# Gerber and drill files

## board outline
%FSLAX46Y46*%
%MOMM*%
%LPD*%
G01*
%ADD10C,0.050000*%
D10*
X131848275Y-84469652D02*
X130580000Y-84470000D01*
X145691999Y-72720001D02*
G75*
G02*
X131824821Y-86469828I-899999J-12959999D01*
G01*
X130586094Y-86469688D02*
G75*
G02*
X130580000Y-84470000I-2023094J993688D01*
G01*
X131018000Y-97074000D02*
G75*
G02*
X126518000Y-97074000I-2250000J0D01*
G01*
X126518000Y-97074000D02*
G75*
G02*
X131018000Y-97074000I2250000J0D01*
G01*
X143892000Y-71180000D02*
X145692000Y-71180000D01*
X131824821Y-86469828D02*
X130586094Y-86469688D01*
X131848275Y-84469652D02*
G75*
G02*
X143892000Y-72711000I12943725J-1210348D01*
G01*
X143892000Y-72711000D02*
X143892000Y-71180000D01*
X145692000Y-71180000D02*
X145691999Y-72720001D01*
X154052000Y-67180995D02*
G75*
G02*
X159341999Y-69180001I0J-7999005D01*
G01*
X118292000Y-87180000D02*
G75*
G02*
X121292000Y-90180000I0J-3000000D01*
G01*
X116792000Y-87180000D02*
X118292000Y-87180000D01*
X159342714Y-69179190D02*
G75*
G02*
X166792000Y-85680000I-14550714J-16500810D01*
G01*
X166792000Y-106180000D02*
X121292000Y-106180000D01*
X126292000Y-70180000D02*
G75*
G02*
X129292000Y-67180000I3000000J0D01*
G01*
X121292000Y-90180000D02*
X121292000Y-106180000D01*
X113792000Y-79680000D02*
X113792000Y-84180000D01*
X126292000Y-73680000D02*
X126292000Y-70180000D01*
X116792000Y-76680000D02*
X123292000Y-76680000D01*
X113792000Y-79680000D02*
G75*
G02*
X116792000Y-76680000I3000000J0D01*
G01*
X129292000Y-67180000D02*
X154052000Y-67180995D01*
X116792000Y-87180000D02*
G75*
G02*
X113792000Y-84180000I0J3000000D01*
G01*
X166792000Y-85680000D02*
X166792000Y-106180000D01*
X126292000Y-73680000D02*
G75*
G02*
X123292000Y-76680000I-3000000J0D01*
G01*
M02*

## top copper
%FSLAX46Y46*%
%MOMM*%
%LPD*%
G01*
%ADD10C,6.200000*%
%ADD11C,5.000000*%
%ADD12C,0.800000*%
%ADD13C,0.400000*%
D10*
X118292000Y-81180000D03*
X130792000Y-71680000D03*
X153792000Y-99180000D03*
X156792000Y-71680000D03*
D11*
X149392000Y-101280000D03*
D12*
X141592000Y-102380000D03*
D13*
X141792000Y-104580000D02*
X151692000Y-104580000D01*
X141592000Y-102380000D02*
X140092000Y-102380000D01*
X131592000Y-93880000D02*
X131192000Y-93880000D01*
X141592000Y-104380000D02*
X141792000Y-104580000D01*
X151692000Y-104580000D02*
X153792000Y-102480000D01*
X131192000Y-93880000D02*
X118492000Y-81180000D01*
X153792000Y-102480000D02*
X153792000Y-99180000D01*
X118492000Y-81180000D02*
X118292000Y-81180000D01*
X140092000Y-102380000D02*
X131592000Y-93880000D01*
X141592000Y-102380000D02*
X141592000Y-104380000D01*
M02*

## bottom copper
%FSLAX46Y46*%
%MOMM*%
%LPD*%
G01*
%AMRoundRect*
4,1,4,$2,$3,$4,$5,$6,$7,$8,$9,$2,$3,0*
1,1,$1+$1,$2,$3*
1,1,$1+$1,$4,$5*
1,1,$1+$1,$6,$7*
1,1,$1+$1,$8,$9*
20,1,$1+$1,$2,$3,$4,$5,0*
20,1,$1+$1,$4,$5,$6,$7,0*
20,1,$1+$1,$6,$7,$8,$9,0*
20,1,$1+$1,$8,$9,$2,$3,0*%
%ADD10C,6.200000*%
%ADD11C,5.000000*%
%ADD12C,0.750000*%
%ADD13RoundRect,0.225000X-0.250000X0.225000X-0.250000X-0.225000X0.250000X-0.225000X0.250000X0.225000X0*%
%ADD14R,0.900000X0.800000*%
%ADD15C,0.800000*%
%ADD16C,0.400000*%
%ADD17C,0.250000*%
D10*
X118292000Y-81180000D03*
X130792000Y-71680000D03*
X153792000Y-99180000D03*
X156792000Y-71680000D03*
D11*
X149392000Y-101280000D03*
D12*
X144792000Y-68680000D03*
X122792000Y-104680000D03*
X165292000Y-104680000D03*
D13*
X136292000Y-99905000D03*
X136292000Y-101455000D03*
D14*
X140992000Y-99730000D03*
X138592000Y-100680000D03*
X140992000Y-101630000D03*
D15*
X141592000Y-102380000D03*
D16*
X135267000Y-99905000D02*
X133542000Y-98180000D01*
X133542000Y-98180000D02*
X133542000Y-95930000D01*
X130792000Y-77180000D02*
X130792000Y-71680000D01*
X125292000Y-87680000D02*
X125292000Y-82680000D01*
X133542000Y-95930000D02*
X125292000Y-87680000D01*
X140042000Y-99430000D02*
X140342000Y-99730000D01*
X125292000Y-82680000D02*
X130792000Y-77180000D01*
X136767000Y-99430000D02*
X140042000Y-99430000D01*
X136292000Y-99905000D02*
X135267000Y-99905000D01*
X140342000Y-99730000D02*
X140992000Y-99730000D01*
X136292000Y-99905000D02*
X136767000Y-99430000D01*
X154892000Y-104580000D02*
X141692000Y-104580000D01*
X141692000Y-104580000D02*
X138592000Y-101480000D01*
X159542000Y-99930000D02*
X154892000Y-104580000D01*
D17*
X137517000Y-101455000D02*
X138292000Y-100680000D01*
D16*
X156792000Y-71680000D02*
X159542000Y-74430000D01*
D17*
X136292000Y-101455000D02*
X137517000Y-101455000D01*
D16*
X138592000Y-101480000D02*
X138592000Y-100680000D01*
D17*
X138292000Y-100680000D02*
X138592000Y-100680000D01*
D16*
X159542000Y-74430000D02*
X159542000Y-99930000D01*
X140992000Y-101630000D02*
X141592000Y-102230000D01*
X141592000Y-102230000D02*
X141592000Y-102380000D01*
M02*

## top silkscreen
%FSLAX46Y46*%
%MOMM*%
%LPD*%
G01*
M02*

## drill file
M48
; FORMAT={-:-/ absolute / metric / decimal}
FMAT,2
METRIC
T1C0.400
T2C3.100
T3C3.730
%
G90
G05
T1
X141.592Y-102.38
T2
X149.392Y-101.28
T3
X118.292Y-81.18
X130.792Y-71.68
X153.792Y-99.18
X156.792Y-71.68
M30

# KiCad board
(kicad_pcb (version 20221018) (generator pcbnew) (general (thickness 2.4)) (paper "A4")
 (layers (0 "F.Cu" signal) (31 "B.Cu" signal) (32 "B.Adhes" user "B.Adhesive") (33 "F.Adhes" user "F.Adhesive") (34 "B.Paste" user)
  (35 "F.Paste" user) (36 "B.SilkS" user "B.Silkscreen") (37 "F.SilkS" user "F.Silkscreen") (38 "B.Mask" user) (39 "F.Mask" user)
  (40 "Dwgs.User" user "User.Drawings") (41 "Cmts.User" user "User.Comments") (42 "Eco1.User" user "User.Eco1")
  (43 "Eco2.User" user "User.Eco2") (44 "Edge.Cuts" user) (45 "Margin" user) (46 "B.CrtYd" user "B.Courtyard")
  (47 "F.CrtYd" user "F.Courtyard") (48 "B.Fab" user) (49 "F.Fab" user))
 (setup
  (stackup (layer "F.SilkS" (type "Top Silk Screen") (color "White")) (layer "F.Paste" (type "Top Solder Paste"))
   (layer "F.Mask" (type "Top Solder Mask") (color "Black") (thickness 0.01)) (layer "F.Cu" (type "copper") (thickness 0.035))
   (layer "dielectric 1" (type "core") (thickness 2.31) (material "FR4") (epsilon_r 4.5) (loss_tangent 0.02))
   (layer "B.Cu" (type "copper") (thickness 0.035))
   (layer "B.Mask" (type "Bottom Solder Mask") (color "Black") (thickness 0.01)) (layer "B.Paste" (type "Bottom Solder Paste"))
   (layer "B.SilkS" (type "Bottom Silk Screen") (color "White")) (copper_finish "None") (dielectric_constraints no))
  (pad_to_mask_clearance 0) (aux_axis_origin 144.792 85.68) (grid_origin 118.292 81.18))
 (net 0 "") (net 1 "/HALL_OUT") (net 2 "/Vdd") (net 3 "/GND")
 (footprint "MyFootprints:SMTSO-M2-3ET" (layer "F.Cu") (at 118.292 81.18 180)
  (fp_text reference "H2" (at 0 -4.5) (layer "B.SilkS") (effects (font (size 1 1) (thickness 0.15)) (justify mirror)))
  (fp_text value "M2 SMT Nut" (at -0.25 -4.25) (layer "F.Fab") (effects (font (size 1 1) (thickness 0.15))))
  (pad "1" thru_hole circle (at 0 0 180) (size 6.2 6.2) (drill 3.73) (layers "*.Cu" "*.Mask" "B.Paste") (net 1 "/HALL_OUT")))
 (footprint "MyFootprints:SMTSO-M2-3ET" (layer "F.Cu") (at 130.792 71.68 180)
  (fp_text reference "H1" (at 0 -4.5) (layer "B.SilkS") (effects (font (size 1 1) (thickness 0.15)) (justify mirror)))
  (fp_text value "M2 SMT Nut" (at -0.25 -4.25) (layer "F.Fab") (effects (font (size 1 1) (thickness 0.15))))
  (pad "1" thru_hole circle (at 0 0 180) (size 6.2 6.2) (drill 3.73) (layers "*.Cu" "*.Mask" "B.Paste") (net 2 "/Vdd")))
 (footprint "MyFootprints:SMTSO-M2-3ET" (layer "F.Cu") (at 153.792 99.18 180)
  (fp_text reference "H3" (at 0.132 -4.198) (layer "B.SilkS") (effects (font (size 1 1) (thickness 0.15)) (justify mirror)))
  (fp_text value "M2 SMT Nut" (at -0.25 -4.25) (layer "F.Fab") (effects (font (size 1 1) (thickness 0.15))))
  (pad "1" thru_hole circle (at 0 0 180) (size 6.2 6.2) (drill 3.73) (layers "*.Cu" "*.Mask" "B.Paste") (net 1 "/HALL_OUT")))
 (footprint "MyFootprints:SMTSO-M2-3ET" (layer "F.Cu") (at 156.792 71.68 180)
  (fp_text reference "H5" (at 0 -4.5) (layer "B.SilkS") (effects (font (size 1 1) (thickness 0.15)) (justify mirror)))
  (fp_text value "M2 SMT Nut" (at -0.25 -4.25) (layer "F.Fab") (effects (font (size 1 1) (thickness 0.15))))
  (pad "1" thru_hole circle (at 0 0 180) (size 6.2 6.2) (drill 3.73) (layers "*.Cu" "*.Mask" "B.Paste") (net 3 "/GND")))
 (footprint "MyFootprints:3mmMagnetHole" (layer "F.Cu") (at 149.392 101.28)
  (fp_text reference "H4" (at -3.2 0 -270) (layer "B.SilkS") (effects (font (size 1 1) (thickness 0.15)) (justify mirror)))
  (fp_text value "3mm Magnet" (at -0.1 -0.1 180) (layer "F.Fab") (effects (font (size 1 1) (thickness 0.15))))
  (pad "1" thru_hole circle (at 0 0) (size 5 5) (drill 3.1) (layers "*.Cu" "*.Mask" "F.Paste")))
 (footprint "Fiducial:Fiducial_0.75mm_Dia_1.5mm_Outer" (layer "B.Cu") (at 144.792 68.68)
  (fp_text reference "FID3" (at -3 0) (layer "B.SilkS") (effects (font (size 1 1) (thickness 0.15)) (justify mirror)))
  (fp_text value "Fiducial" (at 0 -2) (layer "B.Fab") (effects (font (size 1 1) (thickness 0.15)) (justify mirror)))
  (pad "" smd circle (at 0 0) (size 0.75 0.75) (layers "B.Cu" "B.Mask") (solder_mask_margin 0.375) (clearance 0.375)))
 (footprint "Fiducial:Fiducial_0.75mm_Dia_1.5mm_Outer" (layer "B.Cu") (at 122.792 104.68)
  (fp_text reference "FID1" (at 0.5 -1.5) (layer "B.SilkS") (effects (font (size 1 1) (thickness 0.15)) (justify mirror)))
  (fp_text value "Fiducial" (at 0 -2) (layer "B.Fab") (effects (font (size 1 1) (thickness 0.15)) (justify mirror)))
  (pad "" smd circle (at 0 0) (size 0.75 0.75) (layers "B.Cu" "B.Mask") (solder_mask_margin 0.375) (clearance 0.375)))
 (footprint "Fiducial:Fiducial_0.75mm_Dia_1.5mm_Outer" (layer "B.Cu") (at 165.292 104.68)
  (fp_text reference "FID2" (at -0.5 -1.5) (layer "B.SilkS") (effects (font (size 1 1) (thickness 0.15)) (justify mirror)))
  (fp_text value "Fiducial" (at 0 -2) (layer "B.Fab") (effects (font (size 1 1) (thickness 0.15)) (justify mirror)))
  (pad "" smd circle (at 0 0) (size 0.75 0.75) (layers "B.Cu" "B.Mask") (solder_mask_margin 0.375) (clearance 0.375)))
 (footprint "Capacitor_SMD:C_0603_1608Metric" (layer "B.Cu") (at 136.292 100.68 -90)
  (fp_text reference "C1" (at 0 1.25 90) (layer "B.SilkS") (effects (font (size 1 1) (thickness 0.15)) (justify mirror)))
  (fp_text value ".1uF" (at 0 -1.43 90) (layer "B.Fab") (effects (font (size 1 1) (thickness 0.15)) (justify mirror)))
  (pad "1" smd roundrect (at -0.775 0 270) (size 0.9 0.95) (layers "B.Cu" "B.Paste" "B.Mask") (roundrect_rratio 0.25) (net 2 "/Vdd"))
  (pad "2" smd roundrect (at 0.775 0 270) (size 0.9 0.95) (layers "B.Cu" "B.Paste" "B.Mask") (roundrect_rratio 0.25) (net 3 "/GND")))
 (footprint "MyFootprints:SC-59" (layer "B.Cu") (at 139.792 100.68)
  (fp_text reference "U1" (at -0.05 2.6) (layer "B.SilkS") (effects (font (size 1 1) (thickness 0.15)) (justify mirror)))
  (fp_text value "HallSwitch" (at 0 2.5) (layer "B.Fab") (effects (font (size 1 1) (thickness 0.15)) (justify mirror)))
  (pad "1" smd rect (at 1.2 -0.95 180) (size 0.9 0.8) (layers "B.Cu" "B.Paste" "B.Mask") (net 2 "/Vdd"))
  (pad "2" smd rect (at -1.2 0 180) (size 0.9 0.8) (layers "B.Cu" "B.Paste" "B.Mask") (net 3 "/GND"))
  (pad "3" smd rect (at 1.2 0.95 180) (size 0.9 0.8) (layers "B.Cu" "B.Paste" "B.Mask") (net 1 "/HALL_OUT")))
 (gr_line (start 131.848275 84.469652) (end 130.58 84.47) (stroke (width 0.05) (type solid)) (layer "Edge.Cuts"))
 (gr_arc (start 145.691999 72.720001) (mid 153.939058 94.905124) (end 131.824821 86.469828) (stroke (width 0.05) (type solid))
  (layer "Edge.Cuts"))
 (gr_arc (start 130.586094 86.469688) (mid 126.309053 85.482869) (end 130.58 84.47) (stroke (width 0.05) (type solid)) (layer "Edge.Cuts"))
 (gr_circle (center 128.768 97.074) (end 131.018 97.074) (stroke (width 0.05) (type solid)) (fill none) (layer "Edge.Cuts"))
 (gr_line (start 143.892 71.18) (end 145.692 71.18) (stroke (width 0.05) (type solid)) (layer "Edge.Cuts"))
 (gr_line (start 131.824821 86.469828) (end 130.586094 86.469688) (stroke (width 0.05) (type solid)) (layer "Edge.Cuts"))
 (gr_arc (start 131.848275 84.469652) (mid 135.710224 76.378048) (end 143.892 72.711) (stroke (width 0.05) (type solid)) (layer "Edge.Cuts"))
 (gr_line (start 143.892 72.711) (end 143.892 71.18) (stroke (width 0.05) (type solid)) (layer "Edge.Cuts"))
 (gr_line (start 145.692 71.18) (end 145.691999 72.720001) (stroke (width 0.05) (type solid)) (layer "Edge.Cuts"))
 (gr_arc (start 154.052 67.180995) (mid 156.879548 67.697417) (end 159.341999 69.180001) (stroke (width 0.05) (type solid))
  (layer "Edge.Cuts"))
 (gr_arc (start 118.292 87.18) (mid 120.41332 88.05868) (end 121.292 90.18) (stroke (width 0.05) (type solid)) (layer "Edge.Cuts"))
 (gr_line (start 116.792 87.18) (end 118.292 87.18) (stroke (width 0.05) (type solid)) (layer "Edge.Cuts"))
 (gr_arc (start 159.342714 69.17919) (mid 164.84338 76.62781) (end 166.792 85.68) (stroke (width 0.05) (type solid)) (layer "Edge.Cuts"))
 (gr_line (start 166.792 106.18) (end 121.292 106.18) (stroke (width 0.05) (type solid)) (layer "Edge.Cuts"))
 (gr_arc (start 126.292 70.18) (mid 127.17068 68.05868) (end 129.292 67.18) (stroke (width 0.05) (type solid)) (layer "Edge.Cuts"))
 (gr_line (start 121.292 90.18) (end 121.292 106.18) (stroke (width 0.05) (type solid)) (layer "Edge.Cuts"))
 (gr_line (start 113.792 79.68) (end 113.792 84.18) (stroke (width 0.05) (type solid)) (layer "Edge.Cuts"))
 (gr_line (start 126.292 73.68) (end 126.292 70.18) (stroke (width 0.05) (type solid)) (layer "Edge.Cuts"))
 (gr_line (start 116.792 76.68) (end 123.292 76.68) (stroke (width 0.05) (type solid)) (layer "Edge.Cuts"))
 (gr_arc (start 113.792 79.68) (mid 114.67068 77.55868) (end 116.792 76.68) (stroke (width 0.05) (type solid)) (layer "Edge.Cuts"))
 (gr_line (start 129.292 67.18) (end 154.052 67.180995) (stroke (width 0.05) (type solid)) (layer "Edge.Cuts"))
 (gr_arc (start 116.792 87.18) (mid 114.67068 86.30132) (end 113.792 84.18) (stroke (width 0.05) (type solid)) (layer "Edge.Cuts"))
 (gr_line (start 166.792 85.68) (end 166.792 106.18) (stroke (width 0.05) (type solid)) (layer "Edge.Cuts"))
 (gr_arc (start 126.292 73.68) (mid 125.41332 75.80132) (end 123.292 76.68) (stroke (width 0.05) (type solid)) (layer "Edge.Cuts"))
 (segment (start 135.267 99.905) (end 133.542 98.18) (width 0.4) (layer "B.Cu") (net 2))
 (segment (start 133.542 98.18) (end 133.542 95.93) (width 0.4) (layer "B.Cu") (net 2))
 (segment (start 130.792 77.18) (end 130.792 71.68) (width 0.4) (layer "B.Cu") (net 2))
 (segment (start 125.292 87.68) (end 125.292 82.68) (width 0.4) (layer "B.Cu") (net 2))
 (segment (start 133.542 95.93) (end 125.292 87.68) (width 0.4) (layer "B.Cu") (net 2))
 (segment (start 140.042 99.43) (end 140.342 99.73) (width 0.4) (layer "B.Cu") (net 2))
 (segment (start 125.292 82.68) (end 130.792 77.18) (width 0.4) (layer "B.Cu") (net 2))
 (segment (start 136.767 99.43) (end 140.042 99.43) (width 0.4) (layer "B.Cu") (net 2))
 (segment (start 136.292 99.905) (end 135.267 99.905) (width 0.4) (layer "B.Cu") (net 2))
 (segment (start 140.342 99.73) (end 140.992 99.73) (width 0.4) (layer "B.Cu") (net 2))
 (segment (start 136.292 99.905) (end 136.767 99.43) (width 0.4) (layer "B.Cu") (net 2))
 (segment (start 154.892 104.58) (end 141.692 104.58) (width 0.4) (layer "B.Cu") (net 3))
 (segment (start 141.692 104.58) (end 138.592 101.48) (width 0.4) (layer "B.Cu") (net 3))
 (segment (start 159.542 99.93) (end 154.892 104.58) (width 0.4) (layer "B.Cu") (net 3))
 (segment (start 137.517 101.455) (end 138.292 100.68) (width 0.25) (layer "B.Cu") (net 3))
 (segment (start 156.792 71.68) (end 159.542 74.43) (width 0.4) (layer "B.Cu") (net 3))
 (segment (start 136.292 101.455) (end 137.517 101.455) (width 0.25) (layer "B.Cu") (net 3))
 (segment (start 138.592 101.48) (end 138.592 100.68) (width 0.4) (layer "B.Cu") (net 3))
 (segment (start 138.292 100.68) (end 138.592 100.68) (width 0.25) (layer "B.Cu") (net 3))
 (segment (start 159.542 74.43) (end 159.542 99.93) (width 0.4) (layer "B.Cu") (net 3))
 (segment (start 141.792 104.58) (end 151.692 104.58) (width 0.4) (layer "F.Cu") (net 1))
 (segment (start 141.592 102.38) (end 140.092 102.38) (width 0.4) (layer "F.Cu") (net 1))
 (segment (start 131.592 93.88) (end 131.192 93.88) (width 0.4) (layer "F.Cu") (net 1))
 (segment (start 141.592 104.38) (end 141.792 104.58) (width 0.4) (layer "F.Cu") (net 1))
 (segment (start 151.692 104.58) (end 153.792 102.48) (width 0.4) (layer "F.Cu") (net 1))
 (segment (start 131.192 93.88) (end 118.492 81.18) (width 0.4) (layer "F.Cu") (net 1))
 (segment (start 153.792 102.48) (end 153.792 99.18) (width 0.4) (layer "F.Cu") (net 1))
 (segment (start 118.492 81.18) (end 118.292 81.18) (width 0.4) (layer "F.Cu") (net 1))
 (segment (start 140.092 102.38) (end 131.592 93.88) (width 0.4) (layer "F.Cu") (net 1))
 (segment (start 141.592 102.38) (end 141.592 104.38) (width 0.4) (layer "F.Cu") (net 1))
 (via (at 141.592 102.38) (size 0.8) (drill 0.4) (layers "F.Cu" "B.Cu") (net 1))
 (segment (start 140.992 101.63) (end 141.592 102.23) (width 0.4) (layer "B.Cu") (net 1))
 (segment (start 141.592 102.23) (end 141.592 102.38) (width 0.4) (layer "B.Cu") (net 1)))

